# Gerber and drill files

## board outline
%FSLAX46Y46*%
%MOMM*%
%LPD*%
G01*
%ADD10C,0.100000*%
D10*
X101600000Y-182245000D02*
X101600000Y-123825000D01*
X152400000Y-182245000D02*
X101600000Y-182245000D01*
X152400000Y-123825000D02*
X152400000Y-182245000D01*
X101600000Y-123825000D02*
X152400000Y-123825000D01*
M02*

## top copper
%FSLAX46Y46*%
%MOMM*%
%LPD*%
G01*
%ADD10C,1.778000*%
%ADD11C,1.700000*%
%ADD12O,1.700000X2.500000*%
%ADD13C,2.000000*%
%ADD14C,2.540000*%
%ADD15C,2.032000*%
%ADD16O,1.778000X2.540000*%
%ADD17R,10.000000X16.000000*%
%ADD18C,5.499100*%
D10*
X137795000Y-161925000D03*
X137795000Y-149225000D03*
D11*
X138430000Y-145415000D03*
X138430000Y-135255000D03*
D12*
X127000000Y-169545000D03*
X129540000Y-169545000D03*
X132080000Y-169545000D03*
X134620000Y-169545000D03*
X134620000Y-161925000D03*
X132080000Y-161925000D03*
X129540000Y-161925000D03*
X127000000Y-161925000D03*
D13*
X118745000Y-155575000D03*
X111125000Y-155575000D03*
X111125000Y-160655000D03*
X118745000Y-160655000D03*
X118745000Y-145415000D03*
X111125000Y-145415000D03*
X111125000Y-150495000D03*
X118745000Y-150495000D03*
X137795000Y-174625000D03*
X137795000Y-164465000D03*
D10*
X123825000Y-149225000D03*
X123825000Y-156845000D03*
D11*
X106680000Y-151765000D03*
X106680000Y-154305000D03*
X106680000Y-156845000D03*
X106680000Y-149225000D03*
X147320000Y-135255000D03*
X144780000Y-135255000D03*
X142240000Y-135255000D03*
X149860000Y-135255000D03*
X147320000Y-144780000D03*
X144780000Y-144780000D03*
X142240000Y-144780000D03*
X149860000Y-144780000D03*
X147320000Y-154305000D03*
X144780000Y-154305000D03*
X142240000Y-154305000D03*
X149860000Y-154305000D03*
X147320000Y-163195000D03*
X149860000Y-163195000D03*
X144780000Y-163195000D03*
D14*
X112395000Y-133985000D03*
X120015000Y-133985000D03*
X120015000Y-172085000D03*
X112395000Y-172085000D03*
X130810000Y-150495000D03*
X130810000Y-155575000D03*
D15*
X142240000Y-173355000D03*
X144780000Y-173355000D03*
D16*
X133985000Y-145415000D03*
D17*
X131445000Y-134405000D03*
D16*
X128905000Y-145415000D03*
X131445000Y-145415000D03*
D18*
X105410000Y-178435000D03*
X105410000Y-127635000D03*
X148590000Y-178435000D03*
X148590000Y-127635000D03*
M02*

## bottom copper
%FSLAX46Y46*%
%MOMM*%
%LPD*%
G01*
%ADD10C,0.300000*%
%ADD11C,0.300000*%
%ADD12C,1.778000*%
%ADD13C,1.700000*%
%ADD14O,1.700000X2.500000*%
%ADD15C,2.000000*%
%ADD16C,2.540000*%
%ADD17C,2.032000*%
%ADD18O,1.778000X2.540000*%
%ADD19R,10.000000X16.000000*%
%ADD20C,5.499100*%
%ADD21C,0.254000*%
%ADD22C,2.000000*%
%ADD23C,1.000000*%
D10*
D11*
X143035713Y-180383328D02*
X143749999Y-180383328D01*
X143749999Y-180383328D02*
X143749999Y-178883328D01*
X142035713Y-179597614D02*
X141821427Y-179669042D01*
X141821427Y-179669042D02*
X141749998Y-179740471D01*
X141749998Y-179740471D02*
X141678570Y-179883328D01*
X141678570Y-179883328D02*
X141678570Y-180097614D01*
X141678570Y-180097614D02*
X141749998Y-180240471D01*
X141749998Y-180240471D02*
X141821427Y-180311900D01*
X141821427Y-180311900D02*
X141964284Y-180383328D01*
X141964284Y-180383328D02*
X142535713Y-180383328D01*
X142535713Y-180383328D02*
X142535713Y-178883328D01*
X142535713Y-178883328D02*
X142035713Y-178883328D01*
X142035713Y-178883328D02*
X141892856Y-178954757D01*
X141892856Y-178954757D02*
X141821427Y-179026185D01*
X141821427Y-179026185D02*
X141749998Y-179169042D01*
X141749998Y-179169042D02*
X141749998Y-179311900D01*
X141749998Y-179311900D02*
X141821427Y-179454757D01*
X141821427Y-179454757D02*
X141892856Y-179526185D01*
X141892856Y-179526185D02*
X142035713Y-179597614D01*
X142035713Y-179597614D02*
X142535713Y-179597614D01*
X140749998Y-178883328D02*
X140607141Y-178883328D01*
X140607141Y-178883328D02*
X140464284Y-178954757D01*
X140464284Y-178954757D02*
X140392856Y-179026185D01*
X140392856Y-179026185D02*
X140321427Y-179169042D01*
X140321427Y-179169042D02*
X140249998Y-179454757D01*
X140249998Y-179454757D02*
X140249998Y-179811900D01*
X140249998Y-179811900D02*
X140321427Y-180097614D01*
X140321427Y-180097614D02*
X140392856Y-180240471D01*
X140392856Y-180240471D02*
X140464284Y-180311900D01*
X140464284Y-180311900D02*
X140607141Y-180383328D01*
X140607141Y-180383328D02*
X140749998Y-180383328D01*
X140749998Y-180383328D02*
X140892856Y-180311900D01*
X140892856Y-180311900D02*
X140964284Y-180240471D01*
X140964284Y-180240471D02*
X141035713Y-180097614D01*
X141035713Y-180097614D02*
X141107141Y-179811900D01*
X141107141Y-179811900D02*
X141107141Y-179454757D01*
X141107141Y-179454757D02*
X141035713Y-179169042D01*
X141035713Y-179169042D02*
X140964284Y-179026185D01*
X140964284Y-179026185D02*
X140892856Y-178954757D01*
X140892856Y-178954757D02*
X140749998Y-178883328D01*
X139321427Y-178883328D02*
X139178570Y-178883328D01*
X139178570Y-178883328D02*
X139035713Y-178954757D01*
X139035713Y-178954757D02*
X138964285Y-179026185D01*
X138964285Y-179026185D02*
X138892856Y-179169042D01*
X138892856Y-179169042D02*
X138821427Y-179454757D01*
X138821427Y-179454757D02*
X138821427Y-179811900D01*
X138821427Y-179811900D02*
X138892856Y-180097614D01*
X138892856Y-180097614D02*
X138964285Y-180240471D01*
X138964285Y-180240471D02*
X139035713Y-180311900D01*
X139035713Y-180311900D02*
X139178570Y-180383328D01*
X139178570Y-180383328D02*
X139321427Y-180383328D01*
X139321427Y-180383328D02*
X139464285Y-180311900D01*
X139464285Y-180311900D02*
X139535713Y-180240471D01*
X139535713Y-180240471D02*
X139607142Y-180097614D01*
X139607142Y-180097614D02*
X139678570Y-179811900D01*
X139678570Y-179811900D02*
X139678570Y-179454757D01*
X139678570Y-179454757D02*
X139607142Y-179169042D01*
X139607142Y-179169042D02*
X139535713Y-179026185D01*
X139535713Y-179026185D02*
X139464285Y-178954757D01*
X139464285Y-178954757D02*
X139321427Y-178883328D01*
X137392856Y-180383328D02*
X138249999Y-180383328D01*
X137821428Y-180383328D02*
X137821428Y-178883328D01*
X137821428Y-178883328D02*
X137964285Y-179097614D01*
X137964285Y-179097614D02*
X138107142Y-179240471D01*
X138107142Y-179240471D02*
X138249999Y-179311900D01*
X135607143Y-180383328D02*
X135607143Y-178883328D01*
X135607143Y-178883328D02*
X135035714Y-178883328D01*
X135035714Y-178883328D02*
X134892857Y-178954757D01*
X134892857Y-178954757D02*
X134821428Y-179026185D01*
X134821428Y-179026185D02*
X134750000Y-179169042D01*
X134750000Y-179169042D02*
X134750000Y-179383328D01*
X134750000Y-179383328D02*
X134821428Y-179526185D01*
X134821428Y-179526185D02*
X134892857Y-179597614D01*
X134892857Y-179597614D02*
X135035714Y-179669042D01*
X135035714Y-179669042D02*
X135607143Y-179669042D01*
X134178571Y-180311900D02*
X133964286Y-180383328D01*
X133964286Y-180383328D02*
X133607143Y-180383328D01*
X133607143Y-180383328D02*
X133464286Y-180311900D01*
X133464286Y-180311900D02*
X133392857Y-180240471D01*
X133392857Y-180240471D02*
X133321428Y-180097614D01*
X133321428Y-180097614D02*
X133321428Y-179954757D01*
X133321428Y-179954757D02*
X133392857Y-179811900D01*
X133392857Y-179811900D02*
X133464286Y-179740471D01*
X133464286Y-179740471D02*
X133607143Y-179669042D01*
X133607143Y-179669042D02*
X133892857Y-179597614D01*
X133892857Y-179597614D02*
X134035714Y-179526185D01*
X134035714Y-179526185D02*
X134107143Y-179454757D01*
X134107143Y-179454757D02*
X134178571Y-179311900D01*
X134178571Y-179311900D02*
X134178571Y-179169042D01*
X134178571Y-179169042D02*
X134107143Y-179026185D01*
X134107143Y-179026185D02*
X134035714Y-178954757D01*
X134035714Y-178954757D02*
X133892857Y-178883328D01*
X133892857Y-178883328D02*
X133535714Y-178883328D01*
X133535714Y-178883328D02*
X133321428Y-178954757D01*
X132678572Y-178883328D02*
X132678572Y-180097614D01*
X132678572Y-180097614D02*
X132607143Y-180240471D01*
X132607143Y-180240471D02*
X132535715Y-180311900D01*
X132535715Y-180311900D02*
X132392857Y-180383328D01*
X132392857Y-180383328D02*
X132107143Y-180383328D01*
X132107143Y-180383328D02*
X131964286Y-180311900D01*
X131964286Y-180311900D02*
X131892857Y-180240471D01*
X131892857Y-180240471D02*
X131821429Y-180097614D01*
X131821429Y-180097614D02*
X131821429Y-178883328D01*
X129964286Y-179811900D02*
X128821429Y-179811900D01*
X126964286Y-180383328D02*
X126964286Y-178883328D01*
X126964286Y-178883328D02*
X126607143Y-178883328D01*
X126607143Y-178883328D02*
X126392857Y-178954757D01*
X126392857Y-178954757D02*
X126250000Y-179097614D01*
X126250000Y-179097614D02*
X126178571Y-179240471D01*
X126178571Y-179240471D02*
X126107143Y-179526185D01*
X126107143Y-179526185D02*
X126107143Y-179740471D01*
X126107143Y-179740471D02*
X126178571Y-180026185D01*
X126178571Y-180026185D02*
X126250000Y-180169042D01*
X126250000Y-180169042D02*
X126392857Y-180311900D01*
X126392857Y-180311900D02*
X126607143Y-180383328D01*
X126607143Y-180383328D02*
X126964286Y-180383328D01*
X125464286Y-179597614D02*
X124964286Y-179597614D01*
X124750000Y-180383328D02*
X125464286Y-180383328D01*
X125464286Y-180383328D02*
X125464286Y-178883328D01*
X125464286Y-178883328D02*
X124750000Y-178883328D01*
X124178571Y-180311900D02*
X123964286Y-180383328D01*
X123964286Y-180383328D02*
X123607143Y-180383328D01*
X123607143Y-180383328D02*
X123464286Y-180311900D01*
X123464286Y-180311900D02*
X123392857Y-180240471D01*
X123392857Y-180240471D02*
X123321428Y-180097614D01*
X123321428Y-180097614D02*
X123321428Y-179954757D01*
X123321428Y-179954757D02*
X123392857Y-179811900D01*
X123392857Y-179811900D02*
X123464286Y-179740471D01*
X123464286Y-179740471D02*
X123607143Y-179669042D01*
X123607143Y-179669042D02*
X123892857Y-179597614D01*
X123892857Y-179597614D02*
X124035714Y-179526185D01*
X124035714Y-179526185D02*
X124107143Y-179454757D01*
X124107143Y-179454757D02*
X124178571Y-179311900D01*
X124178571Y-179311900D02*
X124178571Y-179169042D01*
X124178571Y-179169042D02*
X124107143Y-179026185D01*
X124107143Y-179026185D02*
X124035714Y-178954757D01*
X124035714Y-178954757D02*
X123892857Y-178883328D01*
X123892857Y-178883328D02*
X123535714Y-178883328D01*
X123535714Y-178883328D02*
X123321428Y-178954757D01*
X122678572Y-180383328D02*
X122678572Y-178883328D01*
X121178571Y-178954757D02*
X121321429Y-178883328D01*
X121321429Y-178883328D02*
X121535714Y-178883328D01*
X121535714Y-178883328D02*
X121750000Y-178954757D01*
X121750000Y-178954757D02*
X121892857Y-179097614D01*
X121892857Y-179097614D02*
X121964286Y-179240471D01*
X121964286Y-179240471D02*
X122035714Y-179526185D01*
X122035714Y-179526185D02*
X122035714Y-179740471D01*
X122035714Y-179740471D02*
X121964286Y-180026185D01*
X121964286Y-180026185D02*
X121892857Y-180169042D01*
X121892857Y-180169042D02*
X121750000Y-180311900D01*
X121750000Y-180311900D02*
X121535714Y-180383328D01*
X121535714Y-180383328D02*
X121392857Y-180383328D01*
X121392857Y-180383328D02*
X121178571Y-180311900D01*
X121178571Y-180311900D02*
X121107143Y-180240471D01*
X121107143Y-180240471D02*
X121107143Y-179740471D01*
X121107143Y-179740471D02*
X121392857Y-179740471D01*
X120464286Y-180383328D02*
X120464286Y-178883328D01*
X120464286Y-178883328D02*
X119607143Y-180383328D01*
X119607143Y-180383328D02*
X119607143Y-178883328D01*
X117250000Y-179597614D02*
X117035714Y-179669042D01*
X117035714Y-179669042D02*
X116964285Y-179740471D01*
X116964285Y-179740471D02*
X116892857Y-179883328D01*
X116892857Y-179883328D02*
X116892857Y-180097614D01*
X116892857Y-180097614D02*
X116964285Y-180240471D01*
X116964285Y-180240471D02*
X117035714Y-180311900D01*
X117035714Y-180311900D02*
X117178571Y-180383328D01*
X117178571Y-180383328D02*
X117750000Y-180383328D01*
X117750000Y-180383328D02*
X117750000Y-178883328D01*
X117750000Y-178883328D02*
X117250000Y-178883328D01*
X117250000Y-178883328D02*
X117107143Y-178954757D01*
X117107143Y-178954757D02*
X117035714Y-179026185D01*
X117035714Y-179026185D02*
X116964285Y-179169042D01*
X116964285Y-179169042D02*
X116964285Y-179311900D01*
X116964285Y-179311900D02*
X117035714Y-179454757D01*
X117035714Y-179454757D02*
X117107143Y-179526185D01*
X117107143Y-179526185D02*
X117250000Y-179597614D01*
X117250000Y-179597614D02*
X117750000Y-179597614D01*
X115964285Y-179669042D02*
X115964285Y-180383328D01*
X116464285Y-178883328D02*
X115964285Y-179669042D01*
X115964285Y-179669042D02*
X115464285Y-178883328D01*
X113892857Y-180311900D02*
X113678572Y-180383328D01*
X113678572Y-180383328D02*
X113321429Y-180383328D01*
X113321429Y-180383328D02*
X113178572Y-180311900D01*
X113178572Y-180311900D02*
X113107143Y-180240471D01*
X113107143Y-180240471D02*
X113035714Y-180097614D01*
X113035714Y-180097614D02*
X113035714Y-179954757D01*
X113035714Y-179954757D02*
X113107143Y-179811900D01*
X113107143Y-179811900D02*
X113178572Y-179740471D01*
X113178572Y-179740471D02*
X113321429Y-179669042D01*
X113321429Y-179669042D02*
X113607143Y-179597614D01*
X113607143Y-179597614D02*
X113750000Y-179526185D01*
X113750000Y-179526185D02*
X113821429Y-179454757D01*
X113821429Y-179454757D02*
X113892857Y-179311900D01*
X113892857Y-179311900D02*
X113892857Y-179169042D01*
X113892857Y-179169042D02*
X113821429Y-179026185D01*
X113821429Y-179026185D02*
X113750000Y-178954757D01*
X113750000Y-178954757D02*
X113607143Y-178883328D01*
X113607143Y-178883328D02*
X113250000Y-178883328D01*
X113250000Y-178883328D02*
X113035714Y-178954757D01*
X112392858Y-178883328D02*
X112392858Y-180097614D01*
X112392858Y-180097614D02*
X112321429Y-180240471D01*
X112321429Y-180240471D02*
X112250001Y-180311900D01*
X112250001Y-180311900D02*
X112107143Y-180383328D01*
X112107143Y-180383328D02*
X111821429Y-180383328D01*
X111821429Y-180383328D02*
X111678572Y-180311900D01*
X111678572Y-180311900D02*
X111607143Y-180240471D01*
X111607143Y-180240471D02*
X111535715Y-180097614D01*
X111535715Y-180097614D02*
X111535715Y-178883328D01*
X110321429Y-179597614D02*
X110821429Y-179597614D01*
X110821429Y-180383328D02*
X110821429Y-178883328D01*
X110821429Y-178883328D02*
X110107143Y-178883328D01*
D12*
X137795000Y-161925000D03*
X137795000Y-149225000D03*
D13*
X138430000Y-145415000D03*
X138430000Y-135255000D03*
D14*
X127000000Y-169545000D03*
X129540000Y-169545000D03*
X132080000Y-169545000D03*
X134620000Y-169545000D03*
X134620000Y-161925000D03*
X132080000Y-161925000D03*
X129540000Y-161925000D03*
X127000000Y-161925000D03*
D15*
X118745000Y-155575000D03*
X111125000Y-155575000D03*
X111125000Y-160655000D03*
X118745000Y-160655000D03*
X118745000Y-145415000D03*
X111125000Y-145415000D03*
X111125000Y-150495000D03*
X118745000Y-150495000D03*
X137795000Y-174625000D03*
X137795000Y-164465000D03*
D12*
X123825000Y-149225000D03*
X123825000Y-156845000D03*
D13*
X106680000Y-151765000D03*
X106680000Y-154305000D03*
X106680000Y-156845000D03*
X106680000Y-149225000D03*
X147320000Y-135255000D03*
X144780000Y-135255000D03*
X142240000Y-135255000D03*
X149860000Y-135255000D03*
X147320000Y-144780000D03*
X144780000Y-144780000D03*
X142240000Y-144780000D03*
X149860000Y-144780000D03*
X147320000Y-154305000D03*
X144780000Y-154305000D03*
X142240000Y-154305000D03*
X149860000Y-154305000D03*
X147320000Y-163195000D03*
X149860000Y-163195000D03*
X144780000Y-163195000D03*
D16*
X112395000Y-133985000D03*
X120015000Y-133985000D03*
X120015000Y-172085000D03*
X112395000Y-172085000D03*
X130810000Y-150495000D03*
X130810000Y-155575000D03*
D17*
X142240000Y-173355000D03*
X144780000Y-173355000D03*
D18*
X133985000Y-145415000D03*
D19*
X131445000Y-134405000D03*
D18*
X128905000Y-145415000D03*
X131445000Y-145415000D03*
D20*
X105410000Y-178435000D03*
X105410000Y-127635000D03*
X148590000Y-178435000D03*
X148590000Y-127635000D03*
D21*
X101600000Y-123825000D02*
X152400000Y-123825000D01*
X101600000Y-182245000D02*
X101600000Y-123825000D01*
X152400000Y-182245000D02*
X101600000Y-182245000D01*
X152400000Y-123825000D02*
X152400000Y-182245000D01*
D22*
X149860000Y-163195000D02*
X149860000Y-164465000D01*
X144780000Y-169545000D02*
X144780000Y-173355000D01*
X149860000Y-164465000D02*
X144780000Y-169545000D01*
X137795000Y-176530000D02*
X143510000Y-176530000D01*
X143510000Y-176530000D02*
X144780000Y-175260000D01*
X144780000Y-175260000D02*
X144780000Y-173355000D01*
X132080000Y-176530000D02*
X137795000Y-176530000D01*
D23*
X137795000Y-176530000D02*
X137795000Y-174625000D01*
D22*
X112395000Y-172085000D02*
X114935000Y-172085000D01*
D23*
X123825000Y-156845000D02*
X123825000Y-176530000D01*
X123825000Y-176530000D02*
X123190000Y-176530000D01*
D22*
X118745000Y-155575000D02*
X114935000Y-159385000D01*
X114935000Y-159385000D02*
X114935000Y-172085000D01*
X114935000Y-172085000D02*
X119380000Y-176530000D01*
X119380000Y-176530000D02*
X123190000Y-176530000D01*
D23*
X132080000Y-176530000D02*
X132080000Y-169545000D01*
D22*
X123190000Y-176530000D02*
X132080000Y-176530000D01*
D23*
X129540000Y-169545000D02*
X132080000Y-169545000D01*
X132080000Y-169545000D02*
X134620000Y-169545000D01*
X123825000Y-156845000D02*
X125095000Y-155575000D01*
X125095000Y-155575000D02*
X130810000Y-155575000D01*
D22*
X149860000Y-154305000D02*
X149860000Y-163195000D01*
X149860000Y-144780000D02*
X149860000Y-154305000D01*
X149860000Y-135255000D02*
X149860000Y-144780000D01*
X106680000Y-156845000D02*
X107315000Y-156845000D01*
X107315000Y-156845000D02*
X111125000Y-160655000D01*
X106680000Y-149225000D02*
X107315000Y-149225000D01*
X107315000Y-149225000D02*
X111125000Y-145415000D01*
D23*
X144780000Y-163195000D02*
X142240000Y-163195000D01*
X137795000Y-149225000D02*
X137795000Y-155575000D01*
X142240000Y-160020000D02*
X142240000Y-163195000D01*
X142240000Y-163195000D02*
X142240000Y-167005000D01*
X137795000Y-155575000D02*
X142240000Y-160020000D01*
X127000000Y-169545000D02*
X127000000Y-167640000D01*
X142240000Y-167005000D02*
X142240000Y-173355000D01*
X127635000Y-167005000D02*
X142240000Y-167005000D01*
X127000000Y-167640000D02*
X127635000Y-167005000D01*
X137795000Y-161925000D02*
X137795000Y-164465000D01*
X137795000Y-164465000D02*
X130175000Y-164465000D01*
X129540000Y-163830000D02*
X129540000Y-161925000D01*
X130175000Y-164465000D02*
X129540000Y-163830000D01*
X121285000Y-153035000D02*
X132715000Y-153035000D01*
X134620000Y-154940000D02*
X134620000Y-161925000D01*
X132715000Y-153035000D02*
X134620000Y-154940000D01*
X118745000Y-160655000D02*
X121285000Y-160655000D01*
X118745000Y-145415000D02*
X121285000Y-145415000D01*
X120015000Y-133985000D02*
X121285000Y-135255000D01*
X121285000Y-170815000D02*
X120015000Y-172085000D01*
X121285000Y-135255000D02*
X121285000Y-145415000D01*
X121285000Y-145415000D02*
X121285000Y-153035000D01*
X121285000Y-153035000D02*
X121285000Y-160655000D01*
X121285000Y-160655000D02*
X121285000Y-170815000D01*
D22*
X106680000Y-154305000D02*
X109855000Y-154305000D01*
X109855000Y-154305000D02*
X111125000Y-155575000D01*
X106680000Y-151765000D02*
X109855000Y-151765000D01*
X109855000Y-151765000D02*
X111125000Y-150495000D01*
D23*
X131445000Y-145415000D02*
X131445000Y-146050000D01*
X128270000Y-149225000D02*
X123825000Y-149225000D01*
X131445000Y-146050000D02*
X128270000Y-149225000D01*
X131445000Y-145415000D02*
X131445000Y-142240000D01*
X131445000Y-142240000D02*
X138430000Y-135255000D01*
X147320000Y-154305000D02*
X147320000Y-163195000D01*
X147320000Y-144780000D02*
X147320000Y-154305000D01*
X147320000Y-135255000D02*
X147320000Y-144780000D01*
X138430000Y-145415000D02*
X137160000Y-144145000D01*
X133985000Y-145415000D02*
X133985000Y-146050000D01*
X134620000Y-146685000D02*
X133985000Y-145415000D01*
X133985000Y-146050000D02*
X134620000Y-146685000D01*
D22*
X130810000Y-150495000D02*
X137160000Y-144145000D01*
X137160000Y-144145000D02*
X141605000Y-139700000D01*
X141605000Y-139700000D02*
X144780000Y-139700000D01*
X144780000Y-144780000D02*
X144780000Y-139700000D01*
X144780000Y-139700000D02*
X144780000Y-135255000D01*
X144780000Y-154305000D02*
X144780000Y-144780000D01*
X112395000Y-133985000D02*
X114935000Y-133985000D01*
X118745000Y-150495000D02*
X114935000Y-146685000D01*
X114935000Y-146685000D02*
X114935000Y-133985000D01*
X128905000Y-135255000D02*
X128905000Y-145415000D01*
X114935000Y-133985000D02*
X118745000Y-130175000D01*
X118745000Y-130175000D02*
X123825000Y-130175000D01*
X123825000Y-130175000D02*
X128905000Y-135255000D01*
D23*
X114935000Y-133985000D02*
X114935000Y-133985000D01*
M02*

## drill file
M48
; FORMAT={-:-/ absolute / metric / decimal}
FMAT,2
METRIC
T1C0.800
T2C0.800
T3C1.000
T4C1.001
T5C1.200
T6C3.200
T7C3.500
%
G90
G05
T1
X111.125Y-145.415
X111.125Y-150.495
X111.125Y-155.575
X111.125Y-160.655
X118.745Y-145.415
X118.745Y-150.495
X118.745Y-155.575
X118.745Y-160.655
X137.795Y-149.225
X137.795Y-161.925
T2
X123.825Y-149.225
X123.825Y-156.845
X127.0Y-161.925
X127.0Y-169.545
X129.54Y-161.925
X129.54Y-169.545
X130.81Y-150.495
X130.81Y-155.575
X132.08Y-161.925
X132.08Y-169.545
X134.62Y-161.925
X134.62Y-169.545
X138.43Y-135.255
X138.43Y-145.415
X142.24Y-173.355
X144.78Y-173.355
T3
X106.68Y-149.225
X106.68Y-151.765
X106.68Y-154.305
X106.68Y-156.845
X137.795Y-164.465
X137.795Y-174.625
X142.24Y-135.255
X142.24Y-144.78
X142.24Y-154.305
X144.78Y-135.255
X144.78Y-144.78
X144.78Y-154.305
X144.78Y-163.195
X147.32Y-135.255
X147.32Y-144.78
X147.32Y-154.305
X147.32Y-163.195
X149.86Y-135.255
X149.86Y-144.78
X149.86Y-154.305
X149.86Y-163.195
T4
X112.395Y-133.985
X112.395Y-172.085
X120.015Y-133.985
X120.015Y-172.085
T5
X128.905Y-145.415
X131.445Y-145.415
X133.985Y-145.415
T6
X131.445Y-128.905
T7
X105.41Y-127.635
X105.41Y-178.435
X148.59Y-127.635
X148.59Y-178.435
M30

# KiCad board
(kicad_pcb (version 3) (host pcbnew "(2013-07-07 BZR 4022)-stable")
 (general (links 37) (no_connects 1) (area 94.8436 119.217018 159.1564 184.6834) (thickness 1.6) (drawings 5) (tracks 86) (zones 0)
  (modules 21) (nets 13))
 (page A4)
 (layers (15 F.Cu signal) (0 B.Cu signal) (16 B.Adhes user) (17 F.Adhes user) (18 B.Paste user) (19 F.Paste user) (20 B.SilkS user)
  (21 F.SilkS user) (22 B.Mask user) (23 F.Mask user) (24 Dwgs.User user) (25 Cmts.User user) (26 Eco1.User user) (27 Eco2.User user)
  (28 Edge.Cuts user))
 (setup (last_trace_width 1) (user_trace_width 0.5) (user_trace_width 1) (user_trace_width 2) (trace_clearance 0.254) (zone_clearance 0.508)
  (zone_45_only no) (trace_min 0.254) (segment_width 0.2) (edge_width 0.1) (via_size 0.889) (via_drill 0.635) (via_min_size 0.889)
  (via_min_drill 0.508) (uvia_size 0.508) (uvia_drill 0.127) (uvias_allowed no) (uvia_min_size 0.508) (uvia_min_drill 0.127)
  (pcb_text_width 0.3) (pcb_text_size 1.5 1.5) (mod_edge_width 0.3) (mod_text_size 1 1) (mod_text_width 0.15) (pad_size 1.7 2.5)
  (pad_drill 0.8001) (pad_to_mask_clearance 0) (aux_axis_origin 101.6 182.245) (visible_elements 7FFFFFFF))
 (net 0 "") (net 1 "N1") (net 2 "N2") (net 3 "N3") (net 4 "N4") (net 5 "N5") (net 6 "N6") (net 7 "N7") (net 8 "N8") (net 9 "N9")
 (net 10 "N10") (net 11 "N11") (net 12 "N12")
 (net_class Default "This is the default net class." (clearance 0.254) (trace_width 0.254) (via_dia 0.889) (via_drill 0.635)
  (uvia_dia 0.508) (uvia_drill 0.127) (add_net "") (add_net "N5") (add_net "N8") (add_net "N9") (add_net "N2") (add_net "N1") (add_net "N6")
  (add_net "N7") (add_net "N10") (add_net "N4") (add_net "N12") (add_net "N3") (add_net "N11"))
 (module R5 (layer F.Cu) (at 137.795 155.575 90) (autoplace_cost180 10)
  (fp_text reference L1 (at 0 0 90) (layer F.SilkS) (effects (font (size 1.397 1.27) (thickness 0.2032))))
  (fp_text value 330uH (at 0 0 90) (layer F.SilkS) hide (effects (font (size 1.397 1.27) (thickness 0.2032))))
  (pad 1 thru_hole circle (at -6.35 0 90) (size 1.778 1.778) (drill 0.8) (layers *.Cu *.Mask F.SilkS) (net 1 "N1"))
  (pad 2 thru_hole circle (at 6.35 0 90) (size 1.778 1.778) (drill 0.8) (layers *.Cu *.Mask F.SilkS) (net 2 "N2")))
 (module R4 (layer F.Cu) (at 138.43 140.335 90) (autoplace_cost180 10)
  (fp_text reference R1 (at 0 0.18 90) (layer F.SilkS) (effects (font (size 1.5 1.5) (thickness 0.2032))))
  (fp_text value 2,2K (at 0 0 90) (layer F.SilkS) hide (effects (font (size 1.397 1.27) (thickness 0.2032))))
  (pad 1 thru_hole circle (at -5.08 0 90) (size 1.7 1.7) (drill 0.8001) (layers *.Cu *.Mask F.SilkS) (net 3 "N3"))
  (pad 2 thru_hole circle (at 5.08 0 90) (size 1.7 1.7) (drill 0.8001) (layers *.Cu *.Mask F.SilkS) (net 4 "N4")))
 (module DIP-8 (layer F.Cu) (at 130.81 165.735)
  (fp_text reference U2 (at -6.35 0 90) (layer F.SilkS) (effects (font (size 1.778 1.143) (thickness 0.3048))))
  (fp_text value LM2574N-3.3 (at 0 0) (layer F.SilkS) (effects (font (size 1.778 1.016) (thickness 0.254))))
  (pad 1 thru_hole oval (at -3.81 3.81) (size 1.7 2.5) (drill 0.8001) (layers *.Cu *.Mask F.SilkS) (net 2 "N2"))
  (pad 2 thru_hole oval (at -1.27 3.81) (size 1.7 2.5) (drill 0.8001) (layers *.Cu *.Mask F.SilkS) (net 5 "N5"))
  (pad 3 thru_hole oval (at 1.27 3.81) (size 1.7 2.5) (drill 0.8001) (layers *.Cu *.Mask F.SilkS) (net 5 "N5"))
  (pad 4 thru_hole oval (at 3.81 3.81) (size 1.7 2.5) (drill 0.8001) (layers *.Cu *.Mask F.SilkS) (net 5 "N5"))
  (pad 5 thru_hole oval (at 3.81 -3.81) (size 1.7 2.5) (drill 0.8001) (layers *.Cu *.Mask F.SilkS) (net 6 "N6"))
  (pad 6 thru_hole oval (at 1.27 -3.81) (size 1.7 2.5) (drill 0.8001) (layers *.Cu *.Mask F.SilkS))
  (pad 7 thru_hole oval (at -1.27 -3.81) (size 1.7 2.5) (drill 0.8001) (layers *.Cu *.Mask F.SilkS) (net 1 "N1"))
  (pad 8 thru_hole oval (at -3.81 -3.81) (size 1.7 2.5) (drill 0.8001) (layers *.Cu *.Mask F.SilkS)))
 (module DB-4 (layer F.Cu) (at 114.935 158.115 270)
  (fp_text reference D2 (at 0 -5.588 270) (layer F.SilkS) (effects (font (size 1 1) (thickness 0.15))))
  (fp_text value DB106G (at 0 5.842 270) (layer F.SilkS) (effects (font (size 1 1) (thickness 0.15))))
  (pad 1 thru_hole circle (at -2.54 -3.81 270) (size 2 2) (drill 0.8) (layers *.Cu *.Mask F.SilkS) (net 5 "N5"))
  (pad 2 thru_hole circle (at -2.54 3.81 270) (size 2 2) (drill 0.8) (layers *.Cu *.Mask F.SilkS) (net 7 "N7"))
  (pad 3 thru_hole circle (at 2.54 3.81 270) (size 2 2) (drill 0.8) (layers *.Cu *.Mask F.SilkS) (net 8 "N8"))
  (pad 4 thru_hole circle (at 2.54 -3.81 270) (size 2 2) (drill 0.8) (layers *.Cu *.Mask F.SilkS) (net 6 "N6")))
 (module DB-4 (layer F.Cu) (at 114.935 147.955 270)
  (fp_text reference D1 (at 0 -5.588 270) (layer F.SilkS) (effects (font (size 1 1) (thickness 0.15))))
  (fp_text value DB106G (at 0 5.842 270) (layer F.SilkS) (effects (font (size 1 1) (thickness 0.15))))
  (pad 1 thru_hole circle (at -2.54 -3.81 270) (size 2 2) (drill 0.8) (layers *.Cu *.Mask F.SilkS) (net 6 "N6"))
  (pad 2 thru_hole circle (at -2.54 3.81 270) (size 2 2) (drill 0.8) (layers *.Cu *.Mask F.SilkS) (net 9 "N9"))
  (pad 3 thru_hole circle (at 2.54 3.81 270) (size 2 2) (drill 0.8) (layers *.Cu *.Mask F.SilkS) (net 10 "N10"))
  (pad 4 thru_hole circle (at 2.54 -3.81 270) (size 2 2) (drill 0.8) (layers *.Cu *.Mask F.SilkS) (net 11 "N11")))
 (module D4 (layer F.Cu) (at 137.795 169.545 90)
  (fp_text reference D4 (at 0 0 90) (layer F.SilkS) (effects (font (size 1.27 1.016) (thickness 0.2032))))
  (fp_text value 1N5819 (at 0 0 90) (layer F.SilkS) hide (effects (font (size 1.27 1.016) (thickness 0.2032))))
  (pad 1 thru_hole circle (at -5.08 0 90) (size 2 2) (drill 1) (layers *.Cu *.Mask F.SilkS) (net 5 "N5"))
  (pad 2 thru_hole circle (at 5.08 0 90) (size 2 2) (drill 1) (layers *.Cu *.Mask F.SilkS) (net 1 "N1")))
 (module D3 (layer F.Cu) (at 123.825 153.035 90)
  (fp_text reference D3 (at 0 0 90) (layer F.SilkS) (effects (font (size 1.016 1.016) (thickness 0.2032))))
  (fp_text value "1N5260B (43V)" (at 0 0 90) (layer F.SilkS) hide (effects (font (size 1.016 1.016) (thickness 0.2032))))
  (pad 2 thru_hole circle (at 3.81 0 90) (size 1.778 1.778) (drill 0.8001) (layers *.Cu *.Mask F.SilkS) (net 4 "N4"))
  (pad 1 thru_hole circle (at -3.81 0 90) (size 1.778 1.778) (drill 0.8001) (layers *.Cu *.Mask F.SilkS) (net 5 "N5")))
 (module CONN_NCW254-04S (layer F.Cu) (at 106.68 153.035 270)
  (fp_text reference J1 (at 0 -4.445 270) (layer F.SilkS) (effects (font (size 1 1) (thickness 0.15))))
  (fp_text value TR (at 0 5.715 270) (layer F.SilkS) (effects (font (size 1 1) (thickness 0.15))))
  (pad 2 thru_hole circle (at -1.27 0 270) (size 1.7 1.7) (drill 1) (layers *.Cu *.Mask F.SilkS) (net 10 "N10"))
  (pad 3 thru_hole circle (at 1.27 0 270) (size 1.7 1.7) (drill 1) (layers *.Cu *.Mask F.SilkS) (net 7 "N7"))
  (pad 4 thru_hole circle (at 3.81 0 270) (size 1.7 1.7) (drill 1) (layers *.Cu *.Mask F.SilkS) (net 8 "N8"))
  (pad 1 thru_hole circle (at -3.81 0 270) (size 1.7 1.7) (drill 1) (layers *.Cu *.Mask F.SilkS) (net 9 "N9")))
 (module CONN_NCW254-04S (layer F.Cu) (at 146.05 135.255 180)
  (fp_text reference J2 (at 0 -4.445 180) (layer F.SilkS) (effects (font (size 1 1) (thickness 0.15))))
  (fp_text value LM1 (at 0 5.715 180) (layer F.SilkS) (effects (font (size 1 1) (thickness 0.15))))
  (pad 2 thru_hole circle (at -1.27 0 180) (size 1.7 1.7) (drill 1) (layers *.Cu *.Mask F.SilkS) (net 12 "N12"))
  (pad 3 thru_hole circle (at 1.27 0 180) (size 1.7 1.7) (drill 1) (layers *.Cu *.Mask F.SilkS) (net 3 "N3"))
  (pad 4 thru_hole circle (at 3.81 0 180) (size 1.7 1.7) (drill 1) (layers *.Cu *.Mask F.SilkS))
  (pad 1 thru_hole circle (at -3.81 0 180) (size 1.7 1.7) (drill 1) (layers *.Cu *.Mask F.SilkS) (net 5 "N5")))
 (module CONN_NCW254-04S (layer F.Cu) (at 146.05 144.78 180)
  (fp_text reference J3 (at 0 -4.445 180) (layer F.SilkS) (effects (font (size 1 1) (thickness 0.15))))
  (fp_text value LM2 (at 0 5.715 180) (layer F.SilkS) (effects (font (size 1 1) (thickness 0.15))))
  (pad 2 thru_hole circle (at -1.27 0 180) (size 1.7 1.7) (drill 1) (layers *.Cu *.Mask F.SilkS) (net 12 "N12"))
  (pad 3 thru_hole circle (at 1.27 0 180) (size 1.7 1.7) (drill 1) (layers *.Cu *.Mask F.SilkS) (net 3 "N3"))
  (pad 4 thru_hole circle (at 3.81 0 180) (size 1.7 1.7) (drill 1) (layers *.Cu *.Mask F.SilkS))
  (pad 1 thru_hole circle (at -3.81 0 180) (size 1.7 1.7) (drill 1) (layers *.Cu *.Mask F.SilkS) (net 5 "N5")))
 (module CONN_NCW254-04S (layer F.Cu) (at 146.05 154.305 180)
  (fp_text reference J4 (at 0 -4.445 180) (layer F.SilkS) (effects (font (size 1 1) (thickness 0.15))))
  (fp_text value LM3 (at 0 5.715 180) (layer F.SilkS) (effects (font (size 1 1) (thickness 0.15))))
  (pad 2 thru_hole circle (at -1.27 0 180) (size 1.7 1.7) (drill 1) (layers *.Cu *.Mask F.SilkS) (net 12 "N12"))
  (pad 3 thru_hole circle (at 1.27 0 180) (size 1.7 1.7) (drill 1) (layers *.Cu *.Mask F.SilkS) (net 3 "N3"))
  (pad 4 thru_hole circle (at 3.81 0 180) (size 1.7 1.7) (drill 1) (layers *.Cu *.Mask F.SilkS))
  (pad 1 thru_hole circle (at -3.81 0 180) (size 1.7 1.7) (drill 1) (layers *.Cu *.Mask F.SilkS) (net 5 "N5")))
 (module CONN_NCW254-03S (layer F.Cu) (at 147.32 163.195)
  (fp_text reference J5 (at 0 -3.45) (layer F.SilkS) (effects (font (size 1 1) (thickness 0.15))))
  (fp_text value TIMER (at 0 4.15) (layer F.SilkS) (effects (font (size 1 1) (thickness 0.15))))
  (pad 2 thru_hole circle (at 0 0) (size 1.7 1.7) (drill 1) (layers *.Cu *.Mask F.SilkS) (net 12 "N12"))
  (pad 3 thru_hole circle (at 2.54 0) (size 1.7 1.7) (drill 1) (layers *.Cu *.Mask F.SilkS) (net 5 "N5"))
  (pad 1 thru_hole circle (at -2.54 0) (size 1.7 1.7) (drill 1) (layers *.Cu *.Mask F.SilkS) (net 2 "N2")))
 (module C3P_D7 (layer F.Cu) (at 116.205 133.985)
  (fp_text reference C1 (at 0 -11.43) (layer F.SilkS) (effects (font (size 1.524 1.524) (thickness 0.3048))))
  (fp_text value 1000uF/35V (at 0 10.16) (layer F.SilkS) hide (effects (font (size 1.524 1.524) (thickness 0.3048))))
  (pad 1 thru_hole circle (at -3.81 0) (size 2.54 2.54) (drill 1.00076) (layers *.Cu *.Mask F.SilkS) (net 11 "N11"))
  (pad 2 thru_hole circle (at 3.81 0) (size 2.54 2.54) (drill 1.00076) (layers *.Cu *.Mask F.SilkS) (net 6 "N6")))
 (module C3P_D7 (layer F.Cu) (at 116.205 172.085 180)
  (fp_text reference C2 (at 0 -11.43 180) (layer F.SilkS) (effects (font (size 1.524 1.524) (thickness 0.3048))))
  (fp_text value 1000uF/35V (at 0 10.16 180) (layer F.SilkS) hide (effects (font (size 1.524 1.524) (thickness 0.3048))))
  (pad 1 thru_hole circle (at -3.81 0 180) (size 2.54 2.54) (drill 1.00076) (layers *.Cu *.Mask F.SilkS) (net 6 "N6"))
  (pad 2 thru_hole circle (at 3.81 0 180) (size 2.54 2.54) (drill 1.00076) (layers *.Cu *.Mask F.SilkS) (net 5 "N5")))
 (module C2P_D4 (layer F.Cu) (at 130.81 153.035 270)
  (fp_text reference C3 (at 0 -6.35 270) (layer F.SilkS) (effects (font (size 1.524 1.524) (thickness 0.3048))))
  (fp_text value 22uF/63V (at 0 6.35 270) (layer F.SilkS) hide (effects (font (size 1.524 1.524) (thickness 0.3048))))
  (pad 1 thru_hole circle (at -2.54 0 270) (size 2.54 2.54) (drill 0.8001) (layers *.Cu *.Mask F.SilkS) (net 3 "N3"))
  (pad 2 thru_hole circle (at 2.54 0 270) (size 2.54 2.54) (drill 0.8001) (layers *.Cu *.Mask F.SilkS) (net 5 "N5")))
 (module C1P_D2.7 (layer F.Cu) (at 143.51 173.355)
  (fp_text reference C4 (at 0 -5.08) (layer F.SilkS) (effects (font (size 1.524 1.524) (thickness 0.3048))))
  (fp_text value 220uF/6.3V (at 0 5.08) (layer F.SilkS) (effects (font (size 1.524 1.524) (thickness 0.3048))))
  (pad 1 thru_hole circle (at -1.27 0) (size 2.032 2.032) (drill 0.8001) (layers *.Cu *.Mask F.SilkS) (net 2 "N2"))
  (pad 2 thru_hole circle (at 1.27 0) (size 2.032 2.032) (drill 0.8001) (layers *.Cu *.Mask F.SilkS) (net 5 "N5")))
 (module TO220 (layer F.Cu) (at 131.445 145.415 90)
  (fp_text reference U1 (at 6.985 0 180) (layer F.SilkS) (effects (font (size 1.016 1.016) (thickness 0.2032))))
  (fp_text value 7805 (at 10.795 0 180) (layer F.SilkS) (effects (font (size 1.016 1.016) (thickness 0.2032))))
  (pad 3 thru_hole oval (at 0 2.54 90) (size 2.54 1.778) (drill 1.2) (layers *.Cu *.Mask F.SilkS) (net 3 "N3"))
  (pad 4 thru_hole rect (at 16.51 0 90) (size 16 10) (drill 3.2 (offset -5.5 0)) (layers *.SilkS *.Mask F.Cu))
  (pad 1 thru_hole oval (at 0 -2.54 90) (size 2.54 1.778) (drill 1.2) (layers *.Cu *.Mask F.SilkS) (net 11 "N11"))
  (pad 2 thru_hole oval (at 0 0 90) (size 2.54 1.778) (drill 1.2) (layers *.Cu *.Mask F.SilkS) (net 4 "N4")))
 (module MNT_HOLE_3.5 (layer F.Cu) (at 105.41 178.435)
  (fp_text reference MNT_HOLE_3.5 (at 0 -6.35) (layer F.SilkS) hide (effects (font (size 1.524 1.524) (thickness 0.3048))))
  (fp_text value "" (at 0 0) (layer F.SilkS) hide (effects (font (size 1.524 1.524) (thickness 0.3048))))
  (pad "" thru_hole circle (at 0 0) (size 5.4991 5.4991) (drill 3.50012) (layers *.Cu *.Mask F.SilkS)))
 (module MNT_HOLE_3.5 (layer F.Cu) (at 105.41 127.635)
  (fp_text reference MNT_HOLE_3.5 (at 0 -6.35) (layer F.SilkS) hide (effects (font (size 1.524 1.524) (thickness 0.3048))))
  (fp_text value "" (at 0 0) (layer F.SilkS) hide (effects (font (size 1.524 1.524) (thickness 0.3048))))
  (pad "" thru_hole circle (at 0 0) (size 5.4991 5.4991) (drill 3.50012) (layers *.Cu *.Mask F.SilkS)))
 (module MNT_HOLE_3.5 (layer F.Cu) (at 148.59 178.435)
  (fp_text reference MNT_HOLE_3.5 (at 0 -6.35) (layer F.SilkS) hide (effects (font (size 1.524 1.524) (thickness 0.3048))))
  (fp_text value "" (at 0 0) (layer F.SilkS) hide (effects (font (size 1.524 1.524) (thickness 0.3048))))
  (pad "" thru_hole circle (at 0 0) (size 5.4991 5.4991) (drill 3.50012) (layers *.Cu *.Mask F.SilkS)))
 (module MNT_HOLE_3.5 (layer F.Cu) (at 148.59 127.635)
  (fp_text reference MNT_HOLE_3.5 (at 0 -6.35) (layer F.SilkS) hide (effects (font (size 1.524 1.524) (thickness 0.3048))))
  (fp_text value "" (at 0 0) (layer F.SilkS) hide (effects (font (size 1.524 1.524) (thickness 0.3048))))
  (pad "" thru_hole circle (at 0 0) (size 5.4991 5.4991) (drill 3.50012) (layers *.Cu *.Mask F.SilkS)))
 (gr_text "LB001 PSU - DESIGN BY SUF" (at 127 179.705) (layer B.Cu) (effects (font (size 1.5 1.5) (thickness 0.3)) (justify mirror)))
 (gr_line (start 101.6 182.245) (end 101.6 123.825) (angle 90) (layer Edge.Cuts) (width 0.1))
 (gr_line (start 152.4 182.245) (end 101.6 182.245) (angle 90) (layer Edge.Cuts) (width 0.1))
 (gr_line (start 152.4 123.825) (end 152.4 182.245) (angle 90) (layer Edge.Cuts) (width 0.1))
 (gr_line (start 101.6 123.825) (end 152.4 123.825) (angle 90) (layer Edge.Cuts) (width 0.1))
 (segment (start 101.6 123.825) (end 152.4 123.825) (width 0.254) (layer B.Cu) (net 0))
 (segment (start 101.6 182.245) (end 101.6 123.825) (width 0.254) (layer B.Cu) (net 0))
 (segment (start 152.4 182.245) (end 101.6 182.245) (width 0.254) (layer B.Cu) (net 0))
 (segment (start 152.4 123.825) (end 152.4 182.245) (width 0.254) (layer B.Cu) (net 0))
 (segment (start 149.86 163.195) (end 149.86 164.465) (width 2) (layer B.Cu) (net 5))
 (segment (start 144.78 169.545) (end 144.78 173.355) (width 2) (layer B.Cu) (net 5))
 (segment (start 149.86 164.465) (end 144.78 169.545) (width 2) (layer B.Cu) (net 5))
 (segment (start 137.795 176.53) (end 143.51 176.53) (width 2) (layer B.Cu) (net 5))
 (segment (start 143.51 176.53) (end 144.78 175.26) (width 2) (layer B.Cu) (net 5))
 (segment (start 144.78 175.26) (end 144.78 173.355) (width 2) (layer B.Cu) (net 5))
 (segment (start 132.08 176.53) (end 137.795 176.53) (width 2) (layer B.Cu) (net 5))
 (segment (start 137.795 176.53) (end 137.795 174.625) (width 1) (layer B.Cu) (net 5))
 (segment (start 112.395 172.085) (end 114.935 172.085) (width 2) (layer B.Cu) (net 5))
 (segment (start 123.825 156.845) (end 123.825 176.53) (width 1) (layer B.Cu) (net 5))
 (segment (start 123.825 176.53) (end 123.19 176.53) (width 1) (layer B.Cu) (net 5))
 (segment (start 118.745 155.575) (end 114.935 159.385) (width 2) (layer B.Cu) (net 5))
 (segment (start 114.935 159.385) (end 114.935 172.085) (width 2) (layer B.Cu) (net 5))
 (segment (start 114.935 172.085) (end 119.38 176.53) (width 2) (layer B.Cu) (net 5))
 (segment (start 119.38 176.53) (end 123.19 176.53) (width 2) (layer B.Cu) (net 5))
 (segment (start 132.08 176.53) (end 132.08 169.545) (width 1) (layer B.Cu) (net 5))
 (segment (start 123.19 176.53) (end 132.08 176.53) (width 2) (layer B.Cu) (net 5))
 (segment (start 129.54 169.545) (end 132.08 169.545) (width 1) (layer B.Cu) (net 5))
 (segment (start 132.08 169.545) (end 134.62 169.545) (width 1) (layer B.Cu) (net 5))
 (segment (start 123.825 156.845) (end 125.095 155.575) (width 1) (layer B.Cu) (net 5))
 (segment (start 125.095 155.575) (end 130.81 155.575) (width 1) (layer B.Cu) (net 5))
 (segment (start 149.86 154.305) (end 149.86 163.195) (width 2) (layer B.Cu) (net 5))
 (segment (start 149.86 144.78) (end 149.86 154.305) (width 2) (layer B.Cu) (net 5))
 (segment (start 149.86 135.255) (end 149.86 144.78) (width 2) (layer B.Cu) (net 5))
 (segment (start 106.68 156.845) (end 107.315 156.845) (width 2) (layer B.Cu) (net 8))
 (segment (start 107.315 156.845) (end 111.125 160.655) (width 2) (layer B.Cu) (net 8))
 (segment (start 106.68 149.225) (end 107.315 149.225) (width 2) (layer B.Cu) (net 9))
 (segment (start 107.315 149.225) (end 111.125 145.415) (width 2) (layer B.Cu) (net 9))
 (segment (start 144.78 163.195) (end 142.24 163.195) (width 1) (layer B.Cu) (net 2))
 (segment (start 137.795 149.225) (end 137.795 155.575) (width 1) (layer B.Cu) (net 2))
 (segment (start 142.24 160.02) (end 142.24 163.195) (width 1) (layer B.Cu) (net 2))
 (segment (start 142.24 163.195) (end 142.24 167.005) (width 1) (layer B.Cu) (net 2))
 (segment (start 137.795 155.575) (end 142.24 160.02) (width 1) (layer B.Cu) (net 2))
 (segment (start 127 169.545) (end 127 167.64) (width 1) (layer B.Cu) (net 2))
 (segment (start 142.24 167.005) (end 142.24 173.355) (width 1) (layer B.Cu) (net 2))
 (segment (start 127.635 167.005) (end 142.24 167.005) (width 1) (layer B.Cu) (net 2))
 (segment (start 127 167.64) (end 127.635 167.005) (width 1) (layer B.Cu) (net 2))
 (segment (start 137.795 161.925) (end 137.795 164.465) (width 1) (layer B.Cu) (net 1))
 (segment (start 137.795 164.465) (end 130.175 164.465) (width 1) (layer B.Cu) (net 1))
 (segment (start 129.54 163.83) (end 129.54 161.925) (width 1) (layer B.Cu) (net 1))
 (segment (start 130.175 164.465) (end 129.54 163.83) (width 1) (layer B.Cu) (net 1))
 (segment (start 121.285 153.035) (end 132.715 153.035) (width 1) (layer B.Cu) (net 6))
 (segment (start 134.62 154.94) (end 134.62 161.925) (width 1) (layer B.Cu) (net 6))
 (segment (start 132.715 153.035) (end 134.62 154.94) (width 1) (layer B.Cu) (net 6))
 (segment (start 118.745 160.655) (end 121.285 160.655) (width 1) (layer B.Cu) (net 6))
 (segment (start 118.745 145.415) (end 121.285 145.415) (width 1) (layer B.Cu) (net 6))
 (segment (start 120.015 133.985) (end 121.285 135.255) (width 1) (layer B.Cu) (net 6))
 (segment (start 121.285 170.815) (end 120.015 172.085) (width 1) (layer B.Cu) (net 6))
 (segment (start 121.285 135.255) (end 121.285 145.415) (width 1) (layer B.Cu) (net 6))
 (segment (start 121.285 145.415) (end 121.285 153.035) (width 1) (layer B.Cu) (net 6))
 (segment (start 121.285 153.035) (end 121.285 160.655) (width 1) (layer B.Cu) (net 6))
 (segment (start 121.285 160.655) (end 121.285 170.815) (width 1) (layer B.Cu) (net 6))
 (segment (start 106.68 154.305) (end 109.855 154.305) (width 2) (layer B.Cu) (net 7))
 (segment (start 109.855 154.305) (end 111.125 155.575) (width 2) (layer B.Cu) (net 7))
 (segment (start 106.68 151.765) (end 109.855 151.765) (width 2) (layer B.Cu) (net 10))
 (segment (start 109.855 151.765) (end 111.125 150.495) (width 2) (layer B.Cu) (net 10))
 (segment (start 131.445 145.415) (end 131.445 146.05) (width 1) (layer B.Cu) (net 4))
 (segment (start 128.27 149.225) (end 123.825 149.225) (width 1) (layer B.Cu) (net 4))
 (segment (start 131.445 146.05) (end 128.27 149.225) (width 1) (layer B.Cu) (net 4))
 (segment (start 131.445 145.415) (end 131.445 142.24) (width 1) (layer B.Cu) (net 4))
 (segment (start 131.445 142.24) (end 138.43 135.255) (width 1) (layer B.Cu) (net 4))
 (segment (start 147.32 154.305) (end 147.32 163.195) (width 1) (layer B.Cu) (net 12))
 (segment (start 147.32 144.78) (end 147.32 154.305) (width 1) (layer B.Cu) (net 12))
 (segment (start 147.32 135.255) (end 147.32 144.78) (width 1) (layer B.Cu) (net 12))
 (segment (start 138.43 145.415) (end 137.16 144.145) (width 1) (layer B.Cu) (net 3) (status 400000))
 (segment (start 133.985 145.415) (end 133.985 146.05) (width 1) (layer B.Cu) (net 3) (status C00000))
 (segment (start 134.62 146.685) (end 133.985 145.415) (width 1) (layer B.Cu) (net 3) (status C00000))
 (segment (start 133.985 146.05) (end 134.62 146.685) (width 1) (layer B.Cu) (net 3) (status C00000))
 (segment (start 130.81 150.495) (end 137.16 144.145) (width 2) (layer B.Cu) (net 3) (status 400000))
 (segment (start 137.16 144.145) (end 141.605 139.7) (width 2) (layer B.Cu) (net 3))
 (segment (start 141.605 139.7) (end 144.78 139.7) (width 2) (layer B.Cu) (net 3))
 (segment (start 144.78 144.78) (end 144.78 139.7) (width 2) (layer B.Cu) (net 3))
 (segment (start 144.78 139.7) (end 144.78 135.255) (width 2) (layer B.Cu) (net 3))
 (segment (start 144.78 154.305) (end 144.78 144.78) (width 2) (layer B.Cu) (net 3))
 (segment (start 112.395 133.985) (end 114.935 133.985) (width 2) (layer B.Cu) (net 11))
 (segment (start 118.745 150.495) (end 114.935 146.685) (width 2) (layer B.Cu) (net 11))
 (segment (start 114.935 146.685) (end 114.935 133.985) (width 2) (layer B.Cu) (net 11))
 (segment (start 128.905 135.255) (end 128.905 145.415) (width 2) (layer B.Cu) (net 11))
 (segment (start 114.935 133.985) (end 118.745 130.175) (width 2) (layer B.Cu) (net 11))
 (segment (start 118.745 130.175) (end 123.825 130.175) (width 2) (layer B.Cu) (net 11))
 (segment (start 123.825 130.175) (end 128.905 135.255) (width 2) (layer B.Cu) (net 11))
 (segment (start 114.935 133.985) (end 114.935 133.985) (width 1) (layer B.Cu) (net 11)))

